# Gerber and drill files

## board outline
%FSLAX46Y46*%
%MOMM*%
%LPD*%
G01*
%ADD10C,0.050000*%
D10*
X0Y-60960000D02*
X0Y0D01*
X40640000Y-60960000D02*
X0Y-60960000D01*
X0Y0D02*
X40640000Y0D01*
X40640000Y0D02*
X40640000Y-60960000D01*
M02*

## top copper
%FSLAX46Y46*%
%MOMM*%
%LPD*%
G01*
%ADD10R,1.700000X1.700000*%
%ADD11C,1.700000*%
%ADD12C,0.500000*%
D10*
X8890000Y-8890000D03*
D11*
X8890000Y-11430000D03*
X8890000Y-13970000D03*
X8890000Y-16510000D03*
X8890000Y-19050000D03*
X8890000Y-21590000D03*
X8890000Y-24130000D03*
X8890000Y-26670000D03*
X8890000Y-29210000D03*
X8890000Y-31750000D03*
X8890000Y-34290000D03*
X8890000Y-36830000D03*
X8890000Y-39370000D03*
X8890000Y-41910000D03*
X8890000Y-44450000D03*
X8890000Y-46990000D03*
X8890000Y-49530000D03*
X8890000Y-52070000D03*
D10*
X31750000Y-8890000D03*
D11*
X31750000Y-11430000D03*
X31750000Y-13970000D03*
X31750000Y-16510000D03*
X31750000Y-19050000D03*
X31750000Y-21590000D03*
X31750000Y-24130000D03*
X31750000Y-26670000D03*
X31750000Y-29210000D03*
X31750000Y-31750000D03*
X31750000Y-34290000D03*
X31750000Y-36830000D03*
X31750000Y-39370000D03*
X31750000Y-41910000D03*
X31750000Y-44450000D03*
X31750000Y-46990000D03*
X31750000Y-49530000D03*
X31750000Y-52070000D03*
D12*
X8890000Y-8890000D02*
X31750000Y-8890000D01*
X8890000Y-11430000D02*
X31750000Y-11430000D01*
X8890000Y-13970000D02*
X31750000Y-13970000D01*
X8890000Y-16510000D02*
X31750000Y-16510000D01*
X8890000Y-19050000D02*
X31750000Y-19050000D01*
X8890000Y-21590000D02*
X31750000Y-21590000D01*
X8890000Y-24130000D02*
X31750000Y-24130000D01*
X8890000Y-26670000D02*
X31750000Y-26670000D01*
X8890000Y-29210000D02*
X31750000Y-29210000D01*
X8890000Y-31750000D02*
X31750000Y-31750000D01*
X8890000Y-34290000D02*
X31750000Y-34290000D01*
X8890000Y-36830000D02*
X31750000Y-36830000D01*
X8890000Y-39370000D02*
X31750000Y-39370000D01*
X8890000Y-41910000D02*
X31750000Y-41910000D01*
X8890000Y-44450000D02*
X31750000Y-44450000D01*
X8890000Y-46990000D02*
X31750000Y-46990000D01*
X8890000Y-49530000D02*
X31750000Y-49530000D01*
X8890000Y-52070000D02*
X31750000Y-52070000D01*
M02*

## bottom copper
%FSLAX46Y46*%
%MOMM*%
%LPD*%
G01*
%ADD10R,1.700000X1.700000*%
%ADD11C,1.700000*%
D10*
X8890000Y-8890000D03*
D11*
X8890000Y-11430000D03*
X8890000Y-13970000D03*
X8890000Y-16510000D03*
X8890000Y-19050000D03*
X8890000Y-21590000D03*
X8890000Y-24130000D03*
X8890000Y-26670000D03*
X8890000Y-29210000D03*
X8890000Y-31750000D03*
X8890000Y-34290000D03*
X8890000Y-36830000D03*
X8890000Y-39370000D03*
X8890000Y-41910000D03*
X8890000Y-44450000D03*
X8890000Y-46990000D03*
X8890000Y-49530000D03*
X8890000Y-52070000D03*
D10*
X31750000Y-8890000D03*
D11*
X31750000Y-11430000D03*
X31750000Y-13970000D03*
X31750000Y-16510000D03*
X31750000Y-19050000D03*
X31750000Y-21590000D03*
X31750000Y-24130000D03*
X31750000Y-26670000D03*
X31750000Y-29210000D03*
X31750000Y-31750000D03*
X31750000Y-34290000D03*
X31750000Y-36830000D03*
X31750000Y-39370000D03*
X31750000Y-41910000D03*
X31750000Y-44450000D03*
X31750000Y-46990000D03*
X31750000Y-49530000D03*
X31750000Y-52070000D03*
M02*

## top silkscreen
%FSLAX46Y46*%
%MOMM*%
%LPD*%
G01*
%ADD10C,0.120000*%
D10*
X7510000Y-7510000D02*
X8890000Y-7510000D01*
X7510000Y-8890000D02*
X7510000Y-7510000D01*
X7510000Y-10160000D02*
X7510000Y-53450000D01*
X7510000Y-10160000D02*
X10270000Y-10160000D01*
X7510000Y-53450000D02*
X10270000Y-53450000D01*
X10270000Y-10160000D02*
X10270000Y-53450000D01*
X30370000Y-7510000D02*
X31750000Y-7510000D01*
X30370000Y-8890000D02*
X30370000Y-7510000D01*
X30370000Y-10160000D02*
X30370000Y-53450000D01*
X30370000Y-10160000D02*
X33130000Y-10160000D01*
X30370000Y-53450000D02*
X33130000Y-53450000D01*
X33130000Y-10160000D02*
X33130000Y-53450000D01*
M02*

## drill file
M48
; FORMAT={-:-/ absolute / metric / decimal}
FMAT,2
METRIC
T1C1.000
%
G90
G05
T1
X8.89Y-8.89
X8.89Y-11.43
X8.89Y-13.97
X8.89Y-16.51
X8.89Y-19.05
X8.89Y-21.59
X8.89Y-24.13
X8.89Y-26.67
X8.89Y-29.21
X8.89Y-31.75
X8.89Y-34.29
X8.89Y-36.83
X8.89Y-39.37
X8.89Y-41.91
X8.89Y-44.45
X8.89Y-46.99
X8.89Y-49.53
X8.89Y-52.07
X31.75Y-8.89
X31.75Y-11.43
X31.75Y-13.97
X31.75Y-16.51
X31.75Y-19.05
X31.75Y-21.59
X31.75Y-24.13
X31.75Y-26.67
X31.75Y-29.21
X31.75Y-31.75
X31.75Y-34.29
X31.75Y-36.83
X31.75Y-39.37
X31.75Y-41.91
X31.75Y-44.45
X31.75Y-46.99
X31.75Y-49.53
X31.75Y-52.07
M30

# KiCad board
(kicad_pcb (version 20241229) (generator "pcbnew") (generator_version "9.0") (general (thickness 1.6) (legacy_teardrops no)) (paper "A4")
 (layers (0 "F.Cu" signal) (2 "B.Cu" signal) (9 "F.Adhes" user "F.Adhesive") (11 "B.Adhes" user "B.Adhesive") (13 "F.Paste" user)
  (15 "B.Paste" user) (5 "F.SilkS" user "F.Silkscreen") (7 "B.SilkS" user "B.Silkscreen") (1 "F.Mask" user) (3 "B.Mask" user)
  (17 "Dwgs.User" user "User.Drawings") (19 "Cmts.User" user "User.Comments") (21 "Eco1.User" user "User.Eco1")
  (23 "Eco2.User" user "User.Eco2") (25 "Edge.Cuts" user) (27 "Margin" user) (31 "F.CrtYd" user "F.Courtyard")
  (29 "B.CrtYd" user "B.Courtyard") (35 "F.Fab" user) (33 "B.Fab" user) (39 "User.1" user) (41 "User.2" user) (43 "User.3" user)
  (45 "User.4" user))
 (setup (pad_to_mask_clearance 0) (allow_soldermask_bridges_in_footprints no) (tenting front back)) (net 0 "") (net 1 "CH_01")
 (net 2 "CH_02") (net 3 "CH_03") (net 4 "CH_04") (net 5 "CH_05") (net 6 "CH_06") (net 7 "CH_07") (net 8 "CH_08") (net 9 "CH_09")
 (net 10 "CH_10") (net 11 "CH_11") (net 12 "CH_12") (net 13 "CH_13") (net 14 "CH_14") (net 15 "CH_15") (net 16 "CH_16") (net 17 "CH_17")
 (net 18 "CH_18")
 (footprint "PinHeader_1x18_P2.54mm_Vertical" (layer "F.Cu") (at 8.89 8.89)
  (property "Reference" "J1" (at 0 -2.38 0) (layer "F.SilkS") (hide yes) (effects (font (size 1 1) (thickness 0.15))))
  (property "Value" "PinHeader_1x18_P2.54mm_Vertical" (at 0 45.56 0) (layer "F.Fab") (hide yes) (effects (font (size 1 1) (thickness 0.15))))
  (fp_line (start -1.38 -1.38) (end 0 -1.38) (stroke (width 0.12) (type solid)) (layer "F.SilkS"))
  (fp_line (start -1.38 0) (end -1.38 -1.38) (stroke (width 0.12) (type solid)) (layer "F.SilkS"))
  (fp_line (start -1.38 1.27) (end -1.38 44.56) (stroke (width 0.12) (type solid)) (layer "F.SilkS"))
  (fp_line (start -1.38 1.27) (end 1.38 1.27) (stroke (width 0.12) (type solid)) (layer "F.SilkS"))
  (fp_line (start -1.38 44.56) (end 1.38 44.56) (stroke (width 0.12) (type solid)) (layer "F.SilkS"))
  (fp_line (start 1.38 1.27) (end 1.38 44.56) (stroke (width 0.12) (type solid)) (layer "F.SilkS"))
  (pad "1" thru_hole rect (at 0 0) (size 1.7 1.7) (drill 1) (layers "*.Cu" "*.Mask") (remove_unused_layers no) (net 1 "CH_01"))
  (pad "2" thru_hole circle (at 0 2.54) (size 1.7 1.7) (drill 1) (layers "*.Cu" "*.Mask") (remove_unused_layers no) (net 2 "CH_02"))
  (pad "3" thru_hole circle (at 0 5.08) (size 1.7 1.7) (drill 1) (layers "*.Cu" "*.Mask") (remove_unused_layers no) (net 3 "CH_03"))
  (pad "4" thru_hole circle (at 0 7.62) (size 1.7 1.7) (drill 1) (layers "*.Cu" "*.Mask") (remove_unused_layers no) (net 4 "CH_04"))
  (pad "5" thru_hole circle (at 0 10.16) (size 1.7 1.7) (drill 1) (layers "*.Cu" "*.Mask") (remove_unused_layers no) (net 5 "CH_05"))
  (pad "6" thru_hole circle (at 0 12.7) (size 1.7 1.7) (drill 1) (layers "*.Cu" "*.Mask") (remove_unused_layers no) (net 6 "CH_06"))
  (pad "7" thru_hole circle (at 0 15.24) (size 1.7 1.7) (drill 1) (layers "*.Cu" "*.Mask") (remove_unused_layers no) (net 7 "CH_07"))
  (pad "8" thru_hole circle (at 0 17.78) (size 1.7 1.7) (drill 1) (layers "*.Cu" "*.Mask") (remove_unused_layers no) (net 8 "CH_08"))
  (pad "9" thru_hole circle (at 0 20.32) (size 1.7 1.7) (drill 1) (layers "*.Cu" "*.Mask") (remove_unused_layers no) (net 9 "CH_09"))
  (pad "10" thru_hole circle (at 0 22.86) (size 1.7 1.7) (drill 1) (layers "*.Cu" "*.Mask") (remove_unused_layers no) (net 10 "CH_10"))
  (pad "11" thru_hole circle (at 0 25.4) (size 1.7 1.7) (drill 1) (layers "*.Cu" "*.Mask") (remove_unused_layers no) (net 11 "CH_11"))
  (pad "12" thru_hole circle (at 0 27.94) (size 1.7 1.7) (drill 1) (layers "*.Cu" "*.Mask") (remove_unused_layers no) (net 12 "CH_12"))
  (pad "13" thru_hole circle (at 0 30.48) (size 1.7 1.7) (drill 1) (layers "*.Cu" "*.Mask") (remove_unused_layers no) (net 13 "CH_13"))
  (pad "14" thru_hole circle (at 0 33.02) (size 1.7 1.7) (drill 1) (layers "*.Cu" "*.Mask") (remove_unused_layers no) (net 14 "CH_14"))
  (pad "15" thru_hole circle (at 0 35.56) (size 1.7 1.7) (drill 1) (layers "*.Cu" "*.Mask") (remove_unused_layers no) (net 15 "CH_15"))
  (pad "16" thru_hole circle (at 0 38.1) (size 1.7 1.7) (drill 1) (layers "*.Cu" "*.Mask") (remove_unused_layers no) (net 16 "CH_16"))
  (pad "17" thru_hole circle (at 0 40.64) (size 1.7 1.7) (drill 1) (layers "*.Cu" "*.Mask") (remove_unused_layers no) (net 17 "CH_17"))
  (pad "18" thru_hole circle (at 0 43.18) (size 1.7 1.7) (drill 1) (layers "*.Cu" "*.Mask") (remove_unused_layers no) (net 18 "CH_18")))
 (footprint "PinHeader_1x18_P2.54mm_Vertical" (layer "F.Cu") (at 31.75 8.89)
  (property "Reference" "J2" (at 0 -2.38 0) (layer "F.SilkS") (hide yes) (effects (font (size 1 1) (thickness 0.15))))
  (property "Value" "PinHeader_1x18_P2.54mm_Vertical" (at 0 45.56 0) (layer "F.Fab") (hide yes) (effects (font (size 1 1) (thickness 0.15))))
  (fp_line (start -1.38 -1.38) (end 0 -1.38) (stroke (width 0.12) (type solid)) (layer "F.SilkS"))
  (fp_line (start -1.38 0) (end -1.38 -1.38) (stroke (width 0.12) (type solid)) (layer "F.SilkS"))
  (fp_line (start -1.38 1.27) (end -1.38 44.56) (stroke (width 0.12) (type solid)) (layer "F.SilkS"))
  (fp_line (start -1.38 1.27) (end 1.38 1.27) (stroke (width 0.12) (type solid)) (layer "F.SilkS"))
  (fp_line (start -1.38 44.56) (end 1.38 44.56) (stroke (width 0.12) (type solid)) (layer "F.SilkS"))
  (fp_line (start 1.38 1.27) (end 1.38 44.56) (stroke (width 0.12) (type solid)) (layer "F.SilkS"))
  (pad "1" thru_hole rect (at 0 0) (size 1.7 1.7) (drill 1) (layers "*.Cu" "*.Mask") (remove_unused_layers no) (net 1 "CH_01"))
  (pad "2" thru_hole circle (at 0 2.54) (size 1.7 1.7) (drill 1) (layers "*.Cu" "*.Mask") (remove_unused_layers no) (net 2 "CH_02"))
  (pad "3" thru_hole circle (at 0 5.08) (size 1.7 1.7) (drill 1) (layers "*.Cu" "*.Mask") (remove_unused_layers no) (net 3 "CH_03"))
  (pad "4" thru_hole circle (at 0 7.62) (size 1.7 1.7) (drill 1) (layers "*.Cu" "*.Mask") (remove_unused_layers no) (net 4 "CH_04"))
  (pad "5" thru_hole circle (at 0 10.16) (size 1.7 1.7) (drill 1) (layers "*.Cu" "*.Mask") (remove_unused_layers no) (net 5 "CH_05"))
  (pad "6" thru_hole circle (at 0 12.7) (size 1.7 1.7) (drill 1) (layers "*.Cu" "*.Mask") (remove_unused_layers no) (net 6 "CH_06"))
  (pad "7" thru_hole circle (at 0 15.24) (size 1.7 1.7) (drill 1) (layers "*.Cu" "*.Mask") (remove_unused_layers no) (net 7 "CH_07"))
  (pad "8" thru_hole circle (at 0 17.78) (size 1.7 1.7) (drill 1) (layers "*.Cu" "*.Mask") (remove_unused_layers no) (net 8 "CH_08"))
  (pad "9" thru_hole circle (at 0 20.32) (size 1.7 1.7) (drill 1) (layers "*.Cu" "*.Mask") (remove_unused_layers no) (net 9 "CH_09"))
  (pad "10" thru_hole circle (at 0 22.86) (size 1.7 1.7) (drill 1) (layers "*.Cu" "*.Mask") (remove_unused_layers no) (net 10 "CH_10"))
  (pad "11" thru_hole circle (at 0 25.4) (size 1.7 1.7) (drill 1) (layers "*.Cu" "*.Mask") (remove_unused_layers no) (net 11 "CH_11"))
  (pad "12" thru_hole circle (at 0 27.94) (size 1.7 1.7) (drill 1) (layers "*.Cu" "*.Mask") (remove_unused_layers no) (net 12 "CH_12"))
  (pad "13" thru_hole circle (at 0 30.48) (size 1.7 1.7) (drill 1) (layers "*.Cu" "*.Mask") (remove_unused_layers no) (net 13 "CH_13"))
  (pad "14" thru_hole circle (at 0 33.02) (size 1.7 1.7) (drill 1) (layers "*.Cu" "*.Mask") (remove_unused_layers no) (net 14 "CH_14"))
  (pad "15" thru_hole circle (at 0 35.56) (size 1.7 1.7) (drill 1) (layers "*.Cu" "*.Mask") (remove_unused_layers no) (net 15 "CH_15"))
  (pad "16" thru_hole circle (at 0 38.1) (size 1.7 1.7) (drill 1) (layers "*.Cu" "*.Mask") (remove_unused_layers no) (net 16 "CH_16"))
  (pad "17" thru_hole circle (at 0 40.64) (size 1.7 1.7) (drill 1) (layers "*.Cu" "*.Mask") (remove_unused_layers no) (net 17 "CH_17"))
  (pad "18" thru_hole circle (at 0 43.18) (size 1.7 1.7) (drill 1) (layers "*.Cu" "*.Mask") (remove_unused_layers no) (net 18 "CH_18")))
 (gr_line (start 0 60.96) (end 0 0) (stroke (width 0.05) (type default)) (layer "Edge.Cuts"))
 (gr_line (start 40.64 60.96) (end 0 60.96) (stroke (width 0.05) (type default)) (layer "Edge.Cuts"))
 (gr_line (start 0 0) (end 40.64 0) (stroke (width 0.05) (type default)) (layer "Edge.Cuts"))
 (gr_line (start 40.64 0) (end 40.64 60.96) (stroke (width 0.05) (type default)) (layer "Edge.Cuts"))
 (segment (start 8.89 8.89) (end 31.75 8.89) (width 0.5) (layer "F.Cu") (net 1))
 (segment (start 8.89 11.43) (end 31.75 11.43) (width 0.5) (layer "F.Cu") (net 2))
 (segment (start 8.89 13.97) (end 31.75 13.97) (width 0.5) (layer "F.Cu") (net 3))
 (segment (start 8.89 16.51) (end 31.75 16.51) (width 0.5) (layer "F.Cu") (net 4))
 (segment (start 8.89 19.05) (end 31.75 19.05) (width 0.5) (layer "F.Cu") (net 5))
 (segment (start 8.89 21.59) (end 31.75 21.59) (width 0.5) (layer "F.Cu") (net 6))
 (segment (start 8.89 24.13) (end 31.75 24.13) (width 0.5) (layer "F.Cu") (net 7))
 (segment (start 8.89 26.67) (end 31.75 26.67) (width 0.5) (layer "F.Cu") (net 8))
 (segment (start 8.89 29.21) (end 31.75 29.21) (width 0.5) (layer "F.Cu") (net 9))
 (segment (start 8.89 31.75) (end 31.75 31.75) (width 0.5) (layer "F.Cu") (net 10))
 (segment (start 8.89 34.29) (end 31.75 34.29) (width 0.5) (layer "F.Cu") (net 11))
 (segment (start 8.89 36.83) (end 31.75 36.83) (width 0.5) (layer "F.Cu") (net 12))
 (segment (start 8.89 39.37) (end 31.75 39.37) (width 0.5) (layer "F.Cu") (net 13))
 (segment (start 8.89 41.91) (end 31.75 41.91) (width 0.5) (layer "F.Cu") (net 14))
 (segment (start 8.89 44.45) (end 31.75 44.45) (width 0.5) (layer "F.Cu") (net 15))
 (segment (start 8.89 46.99) (end 31.75 46.99) (width 0.5) (layer "F.Cu") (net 16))
 (segment (start 8.89 49.53) (end 31.75 49.53) (width 0.5) (layer "F.Cu") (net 17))
 (segment (start 8.89 52.07) (end 31.75 52.07) (width 0.5) (layer "F.Cu") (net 18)))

